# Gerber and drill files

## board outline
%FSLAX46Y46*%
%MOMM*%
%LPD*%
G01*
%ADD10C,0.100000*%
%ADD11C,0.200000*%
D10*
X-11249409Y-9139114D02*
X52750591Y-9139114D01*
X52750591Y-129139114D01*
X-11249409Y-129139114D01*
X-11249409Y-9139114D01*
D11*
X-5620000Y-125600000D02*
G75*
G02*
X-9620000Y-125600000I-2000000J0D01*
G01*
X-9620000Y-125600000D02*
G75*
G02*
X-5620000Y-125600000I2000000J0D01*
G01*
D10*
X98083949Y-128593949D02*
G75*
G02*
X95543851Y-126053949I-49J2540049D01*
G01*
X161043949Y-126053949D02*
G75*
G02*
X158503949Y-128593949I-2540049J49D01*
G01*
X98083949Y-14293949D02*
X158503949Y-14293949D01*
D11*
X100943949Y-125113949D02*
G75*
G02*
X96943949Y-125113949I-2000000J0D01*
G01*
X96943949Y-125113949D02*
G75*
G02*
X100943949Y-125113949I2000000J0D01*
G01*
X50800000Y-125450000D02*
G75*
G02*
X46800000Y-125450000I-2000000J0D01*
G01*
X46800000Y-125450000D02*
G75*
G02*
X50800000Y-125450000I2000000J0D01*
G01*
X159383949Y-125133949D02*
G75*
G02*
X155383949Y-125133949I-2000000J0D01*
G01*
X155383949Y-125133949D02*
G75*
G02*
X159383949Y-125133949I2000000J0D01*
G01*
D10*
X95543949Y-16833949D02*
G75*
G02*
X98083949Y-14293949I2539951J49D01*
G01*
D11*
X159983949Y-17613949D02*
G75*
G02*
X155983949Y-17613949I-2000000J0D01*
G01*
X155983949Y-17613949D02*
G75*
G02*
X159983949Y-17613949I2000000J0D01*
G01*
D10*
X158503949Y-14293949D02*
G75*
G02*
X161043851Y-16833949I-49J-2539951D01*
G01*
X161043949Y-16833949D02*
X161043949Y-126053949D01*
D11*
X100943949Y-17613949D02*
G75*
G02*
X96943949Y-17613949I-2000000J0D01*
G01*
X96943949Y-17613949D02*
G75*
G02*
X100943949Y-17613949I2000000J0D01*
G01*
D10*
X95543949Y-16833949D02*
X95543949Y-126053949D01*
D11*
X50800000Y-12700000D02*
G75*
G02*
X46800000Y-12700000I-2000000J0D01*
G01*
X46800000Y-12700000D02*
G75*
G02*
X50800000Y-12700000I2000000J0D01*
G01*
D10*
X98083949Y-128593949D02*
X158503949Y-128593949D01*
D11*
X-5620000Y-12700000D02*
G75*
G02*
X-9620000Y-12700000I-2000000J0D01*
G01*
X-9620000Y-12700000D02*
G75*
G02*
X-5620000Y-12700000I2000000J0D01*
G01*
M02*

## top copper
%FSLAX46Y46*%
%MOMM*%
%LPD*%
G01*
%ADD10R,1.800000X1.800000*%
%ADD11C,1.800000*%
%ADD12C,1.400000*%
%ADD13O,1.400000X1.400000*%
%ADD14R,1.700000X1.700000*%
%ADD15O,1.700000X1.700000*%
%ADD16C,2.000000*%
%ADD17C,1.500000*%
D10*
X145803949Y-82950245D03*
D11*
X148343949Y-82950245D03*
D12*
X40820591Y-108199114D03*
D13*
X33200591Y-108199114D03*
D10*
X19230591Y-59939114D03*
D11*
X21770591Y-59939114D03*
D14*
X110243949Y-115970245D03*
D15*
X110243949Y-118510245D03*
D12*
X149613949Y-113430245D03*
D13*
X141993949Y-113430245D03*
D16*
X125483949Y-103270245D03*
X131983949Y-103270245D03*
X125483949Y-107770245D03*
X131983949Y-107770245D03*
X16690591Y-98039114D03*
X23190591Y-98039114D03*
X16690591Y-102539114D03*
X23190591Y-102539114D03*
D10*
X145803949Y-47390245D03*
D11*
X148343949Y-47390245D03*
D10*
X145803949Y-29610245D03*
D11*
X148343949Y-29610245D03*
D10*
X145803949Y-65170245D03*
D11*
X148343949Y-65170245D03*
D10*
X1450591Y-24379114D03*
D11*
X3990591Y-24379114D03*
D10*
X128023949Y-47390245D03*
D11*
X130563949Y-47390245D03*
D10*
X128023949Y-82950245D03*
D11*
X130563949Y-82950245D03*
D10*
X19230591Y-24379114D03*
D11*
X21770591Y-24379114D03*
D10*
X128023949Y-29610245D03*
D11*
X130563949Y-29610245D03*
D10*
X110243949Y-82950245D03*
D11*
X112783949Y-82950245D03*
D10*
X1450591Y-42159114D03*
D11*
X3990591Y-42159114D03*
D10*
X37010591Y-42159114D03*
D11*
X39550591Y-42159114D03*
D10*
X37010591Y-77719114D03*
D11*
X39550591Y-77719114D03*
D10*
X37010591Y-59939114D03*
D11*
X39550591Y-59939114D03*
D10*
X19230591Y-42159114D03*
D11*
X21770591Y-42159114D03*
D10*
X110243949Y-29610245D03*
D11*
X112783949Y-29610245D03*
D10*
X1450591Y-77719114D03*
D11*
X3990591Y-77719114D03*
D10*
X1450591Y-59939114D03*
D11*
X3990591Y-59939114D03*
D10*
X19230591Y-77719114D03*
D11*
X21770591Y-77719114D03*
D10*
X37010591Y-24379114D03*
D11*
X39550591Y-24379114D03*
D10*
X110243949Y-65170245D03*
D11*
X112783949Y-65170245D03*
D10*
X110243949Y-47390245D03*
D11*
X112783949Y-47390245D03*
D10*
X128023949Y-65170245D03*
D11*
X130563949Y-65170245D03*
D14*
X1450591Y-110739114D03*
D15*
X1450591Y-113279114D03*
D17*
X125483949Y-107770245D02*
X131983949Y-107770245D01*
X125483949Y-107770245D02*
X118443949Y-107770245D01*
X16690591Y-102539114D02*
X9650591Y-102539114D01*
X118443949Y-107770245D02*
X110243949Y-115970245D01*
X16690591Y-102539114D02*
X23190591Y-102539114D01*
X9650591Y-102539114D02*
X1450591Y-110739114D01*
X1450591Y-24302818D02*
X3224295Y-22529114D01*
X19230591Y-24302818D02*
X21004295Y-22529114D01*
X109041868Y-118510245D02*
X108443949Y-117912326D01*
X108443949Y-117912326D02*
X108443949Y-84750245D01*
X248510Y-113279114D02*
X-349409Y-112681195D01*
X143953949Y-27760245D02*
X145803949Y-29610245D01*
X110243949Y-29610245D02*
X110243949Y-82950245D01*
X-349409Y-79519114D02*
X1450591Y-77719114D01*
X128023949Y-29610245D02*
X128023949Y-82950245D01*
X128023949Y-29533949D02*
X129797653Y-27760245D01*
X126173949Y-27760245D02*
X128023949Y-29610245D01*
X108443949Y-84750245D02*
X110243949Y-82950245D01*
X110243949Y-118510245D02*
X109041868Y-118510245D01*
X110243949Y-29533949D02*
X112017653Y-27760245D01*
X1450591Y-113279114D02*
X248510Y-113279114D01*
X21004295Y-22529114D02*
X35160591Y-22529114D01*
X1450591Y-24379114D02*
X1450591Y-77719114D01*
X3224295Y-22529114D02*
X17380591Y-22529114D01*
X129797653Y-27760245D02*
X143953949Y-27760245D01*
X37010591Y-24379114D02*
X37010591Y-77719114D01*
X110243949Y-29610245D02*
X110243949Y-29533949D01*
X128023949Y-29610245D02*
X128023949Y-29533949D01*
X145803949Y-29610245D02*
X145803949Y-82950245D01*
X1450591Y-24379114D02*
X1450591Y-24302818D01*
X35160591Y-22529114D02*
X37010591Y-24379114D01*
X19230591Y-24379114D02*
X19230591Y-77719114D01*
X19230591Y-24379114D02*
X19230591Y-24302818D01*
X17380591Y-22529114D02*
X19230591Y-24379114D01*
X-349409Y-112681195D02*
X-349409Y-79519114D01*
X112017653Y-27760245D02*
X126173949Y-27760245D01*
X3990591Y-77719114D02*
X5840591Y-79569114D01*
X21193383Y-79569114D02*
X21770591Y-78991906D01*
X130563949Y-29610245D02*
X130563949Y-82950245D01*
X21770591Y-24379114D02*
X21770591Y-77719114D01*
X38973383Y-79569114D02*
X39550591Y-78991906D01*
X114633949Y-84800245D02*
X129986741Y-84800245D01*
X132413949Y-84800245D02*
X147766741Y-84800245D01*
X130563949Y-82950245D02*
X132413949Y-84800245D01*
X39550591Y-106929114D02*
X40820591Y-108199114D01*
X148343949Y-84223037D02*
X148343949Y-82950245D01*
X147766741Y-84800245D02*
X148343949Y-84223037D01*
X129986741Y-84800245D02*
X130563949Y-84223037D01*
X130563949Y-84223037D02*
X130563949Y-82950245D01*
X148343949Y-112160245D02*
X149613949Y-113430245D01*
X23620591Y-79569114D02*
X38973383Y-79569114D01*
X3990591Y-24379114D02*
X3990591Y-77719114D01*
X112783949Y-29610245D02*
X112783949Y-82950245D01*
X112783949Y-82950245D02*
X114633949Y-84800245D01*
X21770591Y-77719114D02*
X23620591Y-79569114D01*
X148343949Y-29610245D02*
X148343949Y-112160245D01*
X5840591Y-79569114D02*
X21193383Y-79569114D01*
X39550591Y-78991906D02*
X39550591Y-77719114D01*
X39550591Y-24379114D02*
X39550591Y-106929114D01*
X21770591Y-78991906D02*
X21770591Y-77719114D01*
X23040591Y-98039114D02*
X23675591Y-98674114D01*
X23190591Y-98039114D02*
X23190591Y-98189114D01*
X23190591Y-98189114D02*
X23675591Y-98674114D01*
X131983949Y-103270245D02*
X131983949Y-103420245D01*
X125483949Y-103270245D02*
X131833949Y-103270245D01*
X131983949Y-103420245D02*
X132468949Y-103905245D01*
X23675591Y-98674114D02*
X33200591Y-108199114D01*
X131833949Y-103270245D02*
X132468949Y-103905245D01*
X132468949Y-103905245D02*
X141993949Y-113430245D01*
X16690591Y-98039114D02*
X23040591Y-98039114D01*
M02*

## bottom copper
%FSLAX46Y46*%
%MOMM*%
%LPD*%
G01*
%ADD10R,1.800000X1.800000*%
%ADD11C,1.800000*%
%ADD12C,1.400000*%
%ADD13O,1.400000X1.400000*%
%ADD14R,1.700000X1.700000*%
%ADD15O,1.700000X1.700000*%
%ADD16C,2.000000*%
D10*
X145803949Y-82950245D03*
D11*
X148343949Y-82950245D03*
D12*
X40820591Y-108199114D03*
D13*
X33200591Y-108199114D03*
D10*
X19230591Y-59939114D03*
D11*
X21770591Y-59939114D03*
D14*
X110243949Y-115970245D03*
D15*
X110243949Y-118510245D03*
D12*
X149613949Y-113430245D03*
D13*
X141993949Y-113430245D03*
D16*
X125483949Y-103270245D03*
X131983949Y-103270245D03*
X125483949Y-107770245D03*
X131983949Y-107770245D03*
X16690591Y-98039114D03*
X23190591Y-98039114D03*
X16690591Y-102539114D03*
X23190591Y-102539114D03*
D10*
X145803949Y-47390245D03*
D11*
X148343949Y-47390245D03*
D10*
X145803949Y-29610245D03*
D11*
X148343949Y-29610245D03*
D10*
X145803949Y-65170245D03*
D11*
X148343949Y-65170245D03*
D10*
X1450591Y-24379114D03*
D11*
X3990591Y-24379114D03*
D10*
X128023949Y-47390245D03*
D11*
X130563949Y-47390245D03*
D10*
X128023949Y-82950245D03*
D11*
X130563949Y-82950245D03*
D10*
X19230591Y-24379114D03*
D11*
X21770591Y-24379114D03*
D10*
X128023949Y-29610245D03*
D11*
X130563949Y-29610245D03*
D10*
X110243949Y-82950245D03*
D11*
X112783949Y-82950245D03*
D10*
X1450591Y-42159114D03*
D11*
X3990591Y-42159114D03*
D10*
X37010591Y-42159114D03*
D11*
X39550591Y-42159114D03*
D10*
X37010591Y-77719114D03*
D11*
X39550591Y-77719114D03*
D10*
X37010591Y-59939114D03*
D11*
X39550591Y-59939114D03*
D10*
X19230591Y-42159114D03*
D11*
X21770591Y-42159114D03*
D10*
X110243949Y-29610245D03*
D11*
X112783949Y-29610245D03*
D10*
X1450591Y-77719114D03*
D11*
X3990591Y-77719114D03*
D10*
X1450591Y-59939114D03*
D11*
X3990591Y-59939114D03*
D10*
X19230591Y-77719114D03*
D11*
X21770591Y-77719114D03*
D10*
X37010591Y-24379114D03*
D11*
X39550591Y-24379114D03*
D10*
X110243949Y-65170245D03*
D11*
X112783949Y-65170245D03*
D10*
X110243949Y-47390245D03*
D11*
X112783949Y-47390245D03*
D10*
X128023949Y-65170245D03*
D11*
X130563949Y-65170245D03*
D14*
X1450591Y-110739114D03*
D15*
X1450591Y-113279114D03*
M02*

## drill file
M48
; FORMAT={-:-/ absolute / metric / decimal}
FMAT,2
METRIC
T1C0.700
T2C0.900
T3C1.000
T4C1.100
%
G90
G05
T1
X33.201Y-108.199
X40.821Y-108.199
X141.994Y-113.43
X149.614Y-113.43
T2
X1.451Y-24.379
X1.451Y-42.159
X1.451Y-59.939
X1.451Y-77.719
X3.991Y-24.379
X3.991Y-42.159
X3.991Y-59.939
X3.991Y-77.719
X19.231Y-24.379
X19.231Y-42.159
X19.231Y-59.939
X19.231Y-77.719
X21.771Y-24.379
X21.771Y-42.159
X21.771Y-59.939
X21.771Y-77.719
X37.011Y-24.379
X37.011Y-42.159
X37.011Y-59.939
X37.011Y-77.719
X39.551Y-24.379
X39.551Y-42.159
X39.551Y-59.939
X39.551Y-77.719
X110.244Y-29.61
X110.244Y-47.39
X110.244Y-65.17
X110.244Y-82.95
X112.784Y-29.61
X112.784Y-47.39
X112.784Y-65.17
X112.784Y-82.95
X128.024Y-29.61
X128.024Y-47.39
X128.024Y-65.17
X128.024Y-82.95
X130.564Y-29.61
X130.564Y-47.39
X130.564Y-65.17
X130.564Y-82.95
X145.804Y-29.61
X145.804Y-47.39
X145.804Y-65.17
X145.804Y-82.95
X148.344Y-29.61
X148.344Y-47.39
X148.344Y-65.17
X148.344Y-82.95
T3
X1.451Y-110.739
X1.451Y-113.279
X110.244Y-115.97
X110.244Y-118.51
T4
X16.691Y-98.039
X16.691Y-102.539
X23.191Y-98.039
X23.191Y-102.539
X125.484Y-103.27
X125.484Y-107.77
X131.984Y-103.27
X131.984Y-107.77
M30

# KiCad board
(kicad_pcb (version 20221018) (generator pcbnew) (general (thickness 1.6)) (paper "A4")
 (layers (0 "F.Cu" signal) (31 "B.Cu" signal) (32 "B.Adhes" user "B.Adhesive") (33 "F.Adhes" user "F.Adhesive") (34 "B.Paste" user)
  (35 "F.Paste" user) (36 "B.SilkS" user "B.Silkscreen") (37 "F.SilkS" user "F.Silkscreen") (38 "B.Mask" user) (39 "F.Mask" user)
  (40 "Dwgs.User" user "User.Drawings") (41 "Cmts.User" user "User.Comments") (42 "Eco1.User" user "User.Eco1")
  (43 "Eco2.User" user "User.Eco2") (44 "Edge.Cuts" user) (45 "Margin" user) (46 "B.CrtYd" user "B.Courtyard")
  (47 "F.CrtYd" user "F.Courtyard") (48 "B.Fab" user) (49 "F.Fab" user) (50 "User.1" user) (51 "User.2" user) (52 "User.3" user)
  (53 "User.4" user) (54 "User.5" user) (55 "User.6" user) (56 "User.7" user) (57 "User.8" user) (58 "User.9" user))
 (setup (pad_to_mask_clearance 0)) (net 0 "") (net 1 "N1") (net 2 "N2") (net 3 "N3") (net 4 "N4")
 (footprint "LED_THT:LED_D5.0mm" (layer "F.Cu") (at 145.803949 82.950245)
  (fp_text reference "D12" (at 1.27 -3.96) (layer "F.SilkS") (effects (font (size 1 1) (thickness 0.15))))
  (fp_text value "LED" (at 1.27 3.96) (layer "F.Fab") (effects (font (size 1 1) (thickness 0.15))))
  (pad "1" thru_hole rect (at 0 0) (size 1.8 1.8) (drill 0.9) (layers "*.Cu" "*.Mask") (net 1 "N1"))
  (pad "2" thru_hole circle (at 2.54 0) (size 1.8 1.8) (drill 0.9) (layers "*.Cu" "*.Mask") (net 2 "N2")))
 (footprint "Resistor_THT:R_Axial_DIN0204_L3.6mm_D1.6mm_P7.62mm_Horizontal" (layer "F.Cu") (at 40.820591 108.199114 180)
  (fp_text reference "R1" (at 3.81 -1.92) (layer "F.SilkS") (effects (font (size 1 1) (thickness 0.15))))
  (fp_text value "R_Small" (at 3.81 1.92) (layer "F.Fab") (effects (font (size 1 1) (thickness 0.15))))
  (pad "1" thru_hole circle (at 0 0 180) (size 1.4 1.4) (drill 0.7) (layers "*.Cu" "*.Mask") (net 2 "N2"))
  (pad "2" thru_hole oval (at 7.62 0 180) (size 1.4 1.4) (drill 0.7) (layers "*.Cu" "*.Mask") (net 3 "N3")))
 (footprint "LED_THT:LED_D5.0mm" (layer "F.Cu") (at 19.230591 59.939114)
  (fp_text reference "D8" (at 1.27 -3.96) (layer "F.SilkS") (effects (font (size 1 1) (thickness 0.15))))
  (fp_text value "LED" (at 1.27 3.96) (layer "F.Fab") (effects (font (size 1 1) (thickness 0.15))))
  (pad "1" thru_hole rect (at 0 0) (size 1.8 1.8) (drill 0.9) (layers "*.Cu" "*.Mask") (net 1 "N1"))
  (pad "2" thru_hole circle (at 2.54 0) (size 1.8 1.8) (drill 0.9) (layers "*.Cu" "*.Mask") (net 2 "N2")))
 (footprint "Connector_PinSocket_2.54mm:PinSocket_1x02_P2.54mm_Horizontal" (layer "F.Cu") (at 110.243949 115.970245)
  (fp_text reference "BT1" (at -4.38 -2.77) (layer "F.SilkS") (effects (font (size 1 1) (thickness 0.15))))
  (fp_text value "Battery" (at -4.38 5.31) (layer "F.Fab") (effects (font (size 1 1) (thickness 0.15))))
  (pad "1" thru_hole rect (at 0 0) (size 1.7 1.7) (drill 1) (layers "*.Cu" "*.Mask") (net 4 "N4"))
  (pad "2" thru_hole oval (at 0 2.54) (size 1.7 1.7) (drill 1) (layers "*.Cu" "*.Mask") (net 1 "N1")))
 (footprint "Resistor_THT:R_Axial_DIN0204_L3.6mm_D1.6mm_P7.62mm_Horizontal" (layer "F.Cu") (at 149.613949 113.430245 180)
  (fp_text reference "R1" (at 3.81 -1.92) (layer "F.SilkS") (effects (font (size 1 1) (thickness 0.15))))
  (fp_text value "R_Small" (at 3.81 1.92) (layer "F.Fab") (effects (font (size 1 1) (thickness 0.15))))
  (pad "1" thru_hole circle (at 0 0 180) (size 1.4 1.4) (drill 0.7) (layers "*.Cu" "*.Mask") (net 2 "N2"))
  (pad "2" thru_hole oval (at 7.62 0 180) (size 1.4 1.4) (drill 0.7) (layers "*.Cu" "*.Mask") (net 3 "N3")))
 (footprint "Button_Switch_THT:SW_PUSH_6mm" (layer "F.Cu") (at 125.483949 103.270245)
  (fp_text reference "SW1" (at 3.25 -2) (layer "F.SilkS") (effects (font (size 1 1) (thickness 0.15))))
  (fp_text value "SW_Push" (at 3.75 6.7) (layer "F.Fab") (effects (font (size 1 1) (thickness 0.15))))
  (pad "1" thru_hole circle (at 0 0 90) (size 2 2) (drill 1.1) (layers "*.Cu" "*.Mask") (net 3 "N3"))
  (pad "1" thru_hole circle (at 6.5 0 90) (size 2 2) (drill 1.1) (layers "*.Cu" "*.Mask") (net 3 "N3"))
  (pad "2" thru_hole circle (at 0 4.5 90) (size 2 2) (drill 1.1) (layers "*.Cu" "*.Mask") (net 4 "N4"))
  (pad "2" thru_hole circle (at 6.5 4.5 90) (size 2 2) (drill 1.1) (layers "*.Cu" "*.Mask") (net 4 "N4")))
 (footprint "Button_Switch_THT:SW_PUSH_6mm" (layer "F.Cu") (at 16.690591 98.039114)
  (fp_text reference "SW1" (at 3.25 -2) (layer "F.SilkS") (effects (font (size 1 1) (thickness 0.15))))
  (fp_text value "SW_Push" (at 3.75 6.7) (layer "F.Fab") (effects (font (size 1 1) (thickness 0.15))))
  (pad "1" thru_hole circle (at 0 0 90) (size 2 2) (drill 1.1) (layers "*.Cu" "*.Mask") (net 3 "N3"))
  (pad "1" thru_hole circle (at 6.5 0 90) (size 2 2) (drill 1.1) (layers "*.Cu" "*.Mask") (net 3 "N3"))
  (pad "2" thru_hole circle (at 0 4.5 90) (size 2 2) (drill 1.1) (layers "*.Cu" "*.Mask") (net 4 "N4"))
  (pad "2" thru_hole circle (at 6.5 4.5 90) (size 2 2) (drill 1.1) (layers "*.Cu" "*.Mask") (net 4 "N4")))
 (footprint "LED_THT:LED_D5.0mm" (layer "F.Cu") (at 145.803949 47.390245)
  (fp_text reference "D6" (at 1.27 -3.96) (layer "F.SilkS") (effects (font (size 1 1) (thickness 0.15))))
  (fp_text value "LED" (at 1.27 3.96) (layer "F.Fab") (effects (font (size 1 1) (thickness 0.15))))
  (pad "1" thru_hole rect (at 0 0) (size 1.8 1.8) (drill 0.9) (layers "*.Cu" "*.Mask") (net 1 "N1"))
  (pad "2" thru_hole circle (at 2.54 0) (size 1.8 1.8) (drill 0.9) (layers "*.Cu" "*.Mask") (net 2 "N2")))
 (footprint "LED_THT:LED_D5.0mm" (layer "F.Cu") (at 145.803949 29.610245)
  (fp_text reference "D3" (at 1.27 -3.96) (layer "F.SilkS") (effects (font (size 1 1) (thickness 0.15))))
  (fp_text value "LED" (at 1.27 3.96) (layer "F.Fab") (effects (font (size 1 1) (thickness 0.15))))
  (pad "1" thru_hole rect (at 0 0) (size 1.8 1.8) (drill 0.9) (layers "*.Cu" "*.Mask") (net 1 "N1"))
  (pad "2" thru_hole circle (at 2.54 0) (size 1.8 1.8) (drill 0.9) (layers "*.Cu" "*.Mask") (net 2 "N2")))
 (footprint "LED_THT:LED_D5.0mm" (layer "F.Cu") (at 145.803949 65.170245)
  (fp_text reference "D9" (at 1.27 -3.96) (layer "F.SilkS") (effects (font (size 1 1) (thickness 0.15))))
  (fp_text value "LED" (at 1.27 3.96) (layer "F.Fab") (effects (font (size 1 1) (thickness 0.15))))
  (pad "1" thru_hole rect (at 0 0) (size 1.8 1.8) (drill 0.9) (layers "*.Cu" "*.Mask") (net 1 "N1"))
  (pad "2" thru_hole circle (at 2.54 0) (size 1.8 1.8) (drill 0.9) (layers "*.Cu" "*.Mask") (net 2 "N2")))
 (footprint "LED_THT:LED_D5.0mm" (layer "F.Cu") (at 1.450591 24.379114)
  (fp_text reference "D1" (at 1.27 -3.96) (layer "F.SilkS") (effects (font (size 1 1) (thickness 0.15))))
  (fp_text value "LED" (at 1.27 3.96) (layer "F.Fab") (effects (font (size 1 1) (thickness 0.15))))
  (pad "1" thru_hole rect (at 0 0) (size 1.8 1.8) (drill 0.9) (layers "*.Cu" "*.Mask") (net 1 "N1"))
  (pad "2" thru_hole circle (at 2.54 0) (size 1.8 1.8) (drill 0.9) (layers "*.Cu" "*.Mask") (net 2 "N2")))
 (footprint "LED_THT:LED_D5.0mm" (layer "F.Cu") (at 128.023949 47.390245)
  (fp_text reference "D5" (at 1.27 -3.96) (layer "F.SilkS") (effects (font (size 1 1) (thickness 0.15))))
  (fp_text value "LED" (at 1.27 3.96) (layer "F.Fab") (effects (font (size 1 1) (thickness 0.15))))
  (pad "1" thru_hole rect (at 0 0) (size 1.8 1.8) (drill 0.9) (layers "*.Cu" "*.Mask") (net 1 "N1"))
  (pad "2" thru_hole circle (at 2.54 0) (size 1.8 1.8) (drill 0.9) (layers "*.Cu" "*.Mask") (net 2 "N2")))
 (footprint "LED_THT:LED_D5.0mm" (layer "F.Cu") (at 128.023949 82.950245)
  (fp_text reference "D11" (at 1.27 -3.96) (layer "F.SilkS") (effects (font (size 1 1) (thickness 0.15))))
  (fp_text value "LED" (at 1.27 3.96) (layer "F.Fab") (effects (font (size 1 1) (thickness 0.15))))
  (pad "1" thru_hole rect (at 0 0) (size 1.8 1.8) (drill 0.9) (layers "*.Cu" "*.Mask") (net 1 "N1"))
  (pad "2" thru_hole circle (at 2.54 0) (size 1.8 1.8) (drill 0.9) (layers "*.Cu" "*.Mask") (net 2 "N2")))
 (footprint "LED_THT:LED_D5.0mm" (layer "F.Cu") (at 19.230591 24.379114)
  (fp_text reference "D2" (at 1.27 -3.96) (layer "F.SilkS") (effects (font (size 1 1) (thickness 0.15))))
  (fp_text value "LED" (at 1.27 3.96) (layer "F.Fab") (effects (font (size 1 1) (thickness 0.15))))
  (pad "1" thru_hole rect (at 0 0) (size 1.8 1.8) (drill 0.9) (layers "*.Cu" "*.Mask") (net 1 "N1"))
  (pad "2" thru_hole circle (at 2.54 0) (size 1.8 1.8) (drill 0.9) (layers "*.Cu" "*.Mask") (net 2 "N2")))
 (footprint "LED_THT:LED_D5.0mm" (layer "F.Cu") (at 128.023949 29.610245)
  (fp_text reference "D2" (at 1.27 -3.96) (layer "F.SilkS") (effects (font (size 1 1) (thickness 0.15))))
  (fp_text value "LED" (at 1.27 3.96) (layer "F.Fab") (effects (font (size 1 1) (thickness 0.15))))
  (pad "1" thru_hole rect (at 0 0) (size 1.8 1.8) (drill 0.9) (layers "*.Cu" "*.Mask") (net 1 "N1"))
  (pad "2" thru_hole circle (at 2.54 0) (size 1.8 1.8) (drill 0.9) (layers "*.Cu" "*.Mask") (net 2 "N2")))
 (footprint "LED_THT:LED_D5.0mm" (layer "F.Cu") (at 110.243949 82.950245)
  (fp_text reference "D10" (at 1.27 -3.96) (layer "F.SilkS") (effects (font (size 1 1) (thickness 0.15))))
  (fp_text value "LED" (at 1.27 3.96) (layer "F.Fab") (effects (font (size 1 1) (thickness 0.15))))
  (pad "1" thru_hole rect (at 0 0) (size 1.8 1.8) (drill 0.9) (layers "*.Cu" "*.Mask") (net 1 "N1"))
  (pad "2" thru_hole circle (at 2.54 0) (size 1.8 1.8) (drill 0.9) (layers "*.Cu" "*.Mask") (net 2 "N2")))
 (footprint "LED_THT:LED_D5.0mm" (layer "F.Cu") (at 1.450591 42.159114)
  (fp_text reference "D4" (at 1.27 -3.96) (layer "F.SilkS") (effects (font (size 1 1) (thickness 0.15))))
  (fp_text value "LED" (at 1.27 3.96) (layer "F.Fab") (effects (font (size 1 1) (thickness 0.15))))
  (pad "1" thru_hole rect (at 0 0) (size 1.8 1.8) (drill 0.9) (layers "*.Cu" "*.Mask") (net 1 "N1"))
  (pad "2" thru_hole circle (at 2.54 0) (size 1.8 1.8) (drill 0.9) (layers "*.Cu" "*.Mask") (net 2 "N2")))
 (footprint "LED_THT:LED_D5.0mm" (layer "F.Cu") (at 37.010591 42.159114)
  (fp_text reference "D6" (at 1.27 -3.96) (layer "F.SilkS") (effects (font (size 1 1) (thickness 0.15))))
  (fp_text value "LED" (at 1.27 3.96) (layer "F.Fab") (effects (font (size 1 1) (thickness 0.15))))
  (pad "1" thru_hole rect (at 0 0) (size 1.8 1.8) (drill 0.9) (layers "*.Cu" "*.Mask") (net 1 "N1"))
  (pad "2" thru_hole circle (at 2.54 0) (size 1.8 1.8) (drill 0.9) (layers "*.Cu" "*.Mask") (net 2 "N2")))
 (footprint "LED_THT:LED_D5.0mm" (layer "F.Cu") (at 37.010591 77.719114)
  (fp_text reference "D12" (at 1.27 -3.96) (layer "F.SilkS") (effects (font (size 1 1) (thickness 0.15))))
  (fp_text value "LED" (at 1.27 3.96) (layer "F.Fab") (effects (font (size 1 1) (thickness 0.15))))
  (pad "1" thru_hole rect (at 0 0) (size 1.8 1.8) (drill 0.9) (layers "*.Cu" "*.Mask") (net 1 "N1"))
  (pad "2" thru_hole circle (at 2.54 0) (size 1.8 1.8) (drill 0.9) (layers "*.Cu" "*.Mask") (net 2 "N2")))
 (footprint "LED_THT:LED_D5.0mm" (layer "F.Cu") (at 37.010591 59.939114)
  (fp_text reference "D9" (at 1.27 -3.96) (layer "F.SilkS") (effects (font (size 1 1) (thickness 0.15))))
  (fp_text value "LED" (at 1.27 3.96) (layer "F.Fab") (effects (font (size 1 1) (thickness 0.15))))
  (pad "1" thru_hole rect (at 0 0) (size 1.8 1.8) (drill 0.9) (layers "*.Cu" "*.Mask") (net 1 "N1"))
  (pad "2" thru_hole circle (at 2.54 0) (size 1.8 1.8) (drill 0.9) (layers "*.Cu" "*.Mask") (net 2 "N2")))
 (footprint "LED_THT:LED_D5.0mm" (layer "F.Cu") (at 19.230591 42.159114)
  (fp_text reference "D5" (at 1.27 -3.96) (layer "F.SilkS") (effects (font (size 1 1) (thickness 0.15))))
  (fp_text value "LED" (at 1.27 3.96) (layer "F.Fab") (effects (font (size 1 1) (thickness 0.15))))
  (pad "1" thru_hole rect (at 0 0) (size 1.8 1.8) (drill 0.9) (layers "*.Cu" "*.Mask") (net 1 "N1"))
  (pad "2" thru_hole circle (at 2.54 0) (size 1.8 1.8) (drill 0.9) (layers "*.Cu" "*.Mask") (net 2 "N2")))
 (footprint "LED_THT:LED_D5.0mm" (layer "F.Cu") (at 110.243949 29.610245)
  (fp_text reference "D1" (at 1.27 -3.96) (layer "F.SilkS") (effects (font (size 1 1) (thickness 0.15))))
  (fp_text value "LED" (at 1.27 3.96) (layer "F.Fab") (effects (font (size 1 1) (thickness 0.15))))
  (pad "1" thru_hole rect (at 0 0) (size 1.8 1.8) (drill 0.9) (layers "*.Cu" "*.Mask") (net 1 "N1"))
  (pad "2" thru_hole circle (at 2.54 0) (size 1.8 1.8) (drill 0.9) (layers "*.Cu" "*.Mask") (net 2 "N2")))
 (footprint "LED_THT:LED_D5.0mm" (layer "F.Cu") (at 1.450591 77.719114)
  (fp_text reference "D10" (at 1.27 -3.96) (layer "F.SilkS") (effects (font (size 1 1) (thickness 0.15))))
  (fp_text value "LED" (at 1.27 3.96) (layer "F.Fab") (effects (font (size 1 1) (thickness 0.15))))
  (pad "1" thru_hole rect (at 0 0) (size 1.8 1.8) (drill 0.9) (layers "*.Cu" "*.Mask") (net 1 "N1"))
  (pad "2" thru_hole circle (at 2.54 0) (size 1.8 1.8) (drill 0.9) (layers "*.Cu" "*.Mask") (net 2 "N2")))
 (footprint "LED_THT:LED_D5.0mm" (layer "F.Cu") (at 1.450591 59.939114)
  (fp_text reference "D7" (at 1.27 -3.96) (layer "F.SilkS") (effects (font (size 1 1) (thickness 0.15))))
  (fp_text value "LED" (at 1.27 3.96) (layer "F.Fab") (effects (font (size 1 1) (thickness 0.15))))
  (pad "1" thru_hole rect (at 0 0) (size 1.8 1.8) (drill 0.9) (layers "*.Cu" "*.Mask") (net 1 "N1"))
  (pad "2" thru_hole circle (at 2.54 0) (size 1.8 1.8) (drill 0.9) (layers "*.Cu" "*.Mask") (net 2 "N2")))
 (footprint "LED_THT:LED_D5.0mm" (layer "F.Cu") (at 19.230591 77.719114)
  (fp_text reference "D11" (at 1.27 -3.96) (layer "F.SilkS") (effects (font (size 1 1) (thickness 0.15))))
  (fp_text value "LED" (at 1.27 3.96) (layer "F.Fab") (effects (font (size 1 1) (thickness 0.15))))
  (pad "1" thru_hole rect (at 0 0) (size 1.8 1.8) (drill 0.9) (layers "*.Cu" "*.Mask") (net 1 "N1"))
  (pad "2" thru_hole circle (at 2.54 0) (size 1.8 1.8) (drill 0.9) (layers "*.Cu" "*.Mask") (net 2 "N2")))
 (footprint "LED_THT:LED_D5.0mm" (layer "F.Cu") (at 37.010591 24.379114)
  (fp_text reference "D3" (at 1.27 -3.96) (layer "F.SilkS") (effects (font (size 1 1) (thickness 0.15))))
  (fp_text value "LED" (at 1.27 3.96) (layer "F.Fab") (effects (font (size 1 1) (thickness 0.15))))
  (pad "1" thru_hole rect (at 0 0) (size 1.8 1.8) (drill 0.9) (layers "*.Cu" "*.Mask") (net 1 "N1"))
  (pad "2" thru_hole circle (at 2.54 0) (size 1.8 1.8) (drill 0.9) (layers "*.Cu" "*.Mask") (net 2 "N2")))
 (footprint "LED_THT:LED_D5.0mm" (layer "F.Cu") (at 110.243949 65.170245)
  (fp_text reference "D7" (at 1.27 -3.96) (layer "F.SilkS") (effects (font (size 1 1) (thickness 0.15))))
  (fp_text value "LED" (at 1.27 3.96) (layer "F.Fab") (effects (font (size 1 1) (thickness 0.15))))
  (pad "1" thru_hole rect (at 0 0) (size 1.8 1.8) (drill 0.9) (layers "*.Cu" "*.Mask") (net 1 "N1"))
  (pad "2" thru_hole circle (at 2.54 0) (size 1.8 1.8) (drill 0.9) (layers "*.Cu" "*.Mask") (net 2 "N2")))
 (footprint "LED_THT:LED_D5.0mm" (layer "F.Cu") (at 110.243949 47.390245)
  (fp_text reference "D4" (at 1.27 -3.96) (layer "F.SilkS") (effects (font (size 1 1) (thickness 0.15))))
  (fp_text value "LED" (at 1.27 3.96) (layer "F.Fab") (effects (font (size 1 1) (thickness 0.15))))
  (pad "1" thru_hole rect (at 0 0) (size 1.8 1.8) (drill 0.9) (layers "*.Cu" "*.Mask") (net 1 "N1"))
  (pad "2" thru_hole circle (at 2.54 0) (size 1.8 1.8) (drill 0.9) (layers "*.Cu" "*.Mask") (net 2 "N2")))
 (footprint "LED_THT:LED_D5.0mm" (layer "F.Cu") (at 128.023949 65.170245)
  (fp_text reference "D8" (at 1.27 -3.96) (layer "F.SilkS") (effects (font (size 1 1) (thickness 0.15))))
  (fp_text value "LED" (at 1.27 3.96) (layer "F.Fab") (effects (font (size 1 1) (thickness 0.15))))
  (pad "1" thru_hole rect (at 0 0) (size 1.8 1.8) (drill 0.9) (layers "*.Cu" "*.Mask") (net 1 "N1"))
  (pad "2" thru_hole circle (at 2.54 0) (size 1.8 1.8) (drill 0.9) (layers "*.Cu" "*.Mask") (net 2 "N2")))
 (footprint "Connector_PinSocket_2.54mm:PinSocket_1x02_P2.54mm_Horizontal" (layer "F.Cu") (at 1.450591 110.739114)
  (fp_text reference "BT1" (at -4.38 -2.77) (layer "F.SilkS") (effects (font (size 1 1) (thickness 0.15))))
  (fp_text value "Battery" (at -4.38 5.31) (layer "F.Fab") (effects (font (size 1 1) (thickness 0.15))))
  (pad "1" thru_hole rect (at 0 0) (size 1.7 1.7) (drill 1) (layers "*.Cu" "*.Mask") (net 4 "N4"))
  (pad "2" thru_hole oval (at 0 2.54) (size 1.7 1.7) (drill 1) (layers "*.Cu" "*.Mask") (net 1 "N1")))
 (gr_rect (start -11.249409 9.139114) (end 52.750591 129.139114) (stroke (width 0.1) (type default)) (fill none) (layer "Edge.Cuts"))
 (gr_circle (center -7.62 125.6) (end -5.62 125.6) (stroke (width 0.2) (type default)) (fill none) (layer "Edge.Cuts"))
 (gr_arc (start 98.083949 128.593949) (mid 96.287898 127.85) (end 95.543949 126.053949) (stroke (width 0.1) (type default))
  (layer "Edge.Cuts"))
 (gr_arc (start 161.043949 126.053949) (mid 160.3 127.85) (end 158.503949 128.593949) (stroke (width 0.1) (type default))
  (layer "Edge.Cuts"))
 (gr_line (start 98.083949 14.293949) (end 158.503949 14.293949) (stroke (width 0.1) (type default)) (layer "Edge.Cuts"))
 (gr_circle (center 98.943949 125.113949) (end 96.943949 125.113949) (stroke (width 0.2) (type default)) (fill none) (layer "Edge.Cuts"))
 (gr_circle (center 48.8 125.45) (end 50.8 125.45) (stroke (width 0.2) (type default)) (fill none) (layer "Edge.Cuts"))
 (gr_circle (center 157.383949 125.133949) (end 155.383949 125.133949) (stroke (width 0.2) (type default)) (fill none) (layer "Edge.Cuts"))
 (gr_arc (start 95.543949 16.833949) (mid 96.287898 15.037898) (end 98.083949 14.293949) (stroke (width 0.1) (type default))
  (layer "Edge.Cuts"))
 (gr_circle (center 157.983949 17.613949) (end 155.983949 17.613949) (stroke (width 0.2) (type default)) (fill none) (layer "Edge.Cuts"))
 (gr_arc (start 158.503949 14.293949) (mid 160.3 15.037898) (end 161.043949 16.833949) (stroke (width 0.1) (type default))
  (layer "Edge.Cuts"))
 (gr_line (start 161.043949 16.833949) (end 161.043949 126.053949) (stroke (width 0.1) (type default)) (layer "Edge.Cuts"))
 (gr_circle (center 98.943949 17.613949) (end 96.943949 17.613949) (stroke (width 0.2) (type default)) (fill none) (layer "Edge.Cuts"))
 (gr_line (start 95.543949 16.833949) (end 95.543949 126.053949) (stroke (width 0.1) (type default)) (layer "Edge.Cuts"))
 (gr_circle (center 48.8 12.7) (end 50.8 12.7) (stroke (width 0.2) (type default)) (fill none) (layer "Edge.Cuts"))
 (gr_line (start 98.083949 128.593949) (end 158.503949 128.593949) (stroke (width 0.1) (type default)) (layer "Edge.Cuts"))
 (gr_circle (center -7.62 12.7) (end -5.62 12.7) (stroke (width 0.2) (type default)) (fill none) (layer "Edge.Cuts"))
 (segment (start 125.483949 107.770245) (end 131.983949 107.770245) (width 1.5) (layer "F.Cu") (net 4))
 (segment (start 125.483949 107.770245) (end 118.443949 107.770245) (width 1.5) (layer "F.Cu") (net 4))
 (segment (start 16.690591 102.539114) (end 9.650591 102.539114) (width 1.5) (layer "F.Cu") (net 4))
 (segment (start 118.443949 107.770245) (end 110.243949 115.970245) (width 1.5) (layer "F.Cu") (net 4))
 (segment (start 16.690591 102.539114) (end 23.190591 102.539114) (width 1.5) (layer "F.Cu") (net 4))
 (segment (start 9.650591 102.539114) (end 1.450591 110.739114) (width 1.5) (layer "F.Cu") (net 4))
 (segment (start 1.450591 24.302818) (end 3.224295 22.529114) (width 1.5) (layer "F.Cu") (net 1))
 (segment (start 19.230591 24.302818) (end 21.004295 22.529114) (width 1.5) (layer "F.Cu") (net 1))
 (segment (start 109.041868 118.510245) (end 108.443949 117.912326) (width 1.5) (layer "F.Cu") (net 1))
 (segment (start 108.443949 117.912326) (end 108.443949 84.750245) (width 1.5) (layer "F.Cu") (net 1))
 (segment (start 0.24851 113.279114) (end -0.349409 112.681195) (width 1.5) (layer "F.Cu") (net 1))
 (segment (start 143.953949 27.760245) (end 145.803949 29.610245) (width 1.5) (layer "F.Cu") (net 1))
 (segment (start 110.243949 29.610245) (end 110.243949 82.950245) (width 1.5) (layer "F.Cu") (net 1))
 (segment (start -0.349409 79.519114) (end 1.450591 77.719114) (width 1.5) (layer "F.Cu") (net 1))
 (segment (start 128.023949 29.610245) (end 128.023949 82.950245) (width 1.5) (layer "F.Cu") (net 1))
 (segment (start 128.023949 29.533949) (end 129.797653 27.760245) (width 1.5) (layer "F.Cu") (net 1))
 (segment (start 126.173949 27.760245) (end 128.023949 29.610245) (width 1.5) (layer "F.Cu") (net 1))
 (segment (start 108.443949 84.750245) (end 110.243949 82.950245) (width 1.5) (layer "F.Cu") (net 1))
 (segment (start 110.243949 118.510245) (end 109.041868 118.510245) (width 1.5) (layer "F.Cu") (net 1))
 (segment (start 110.243949 29.533949) (end 112.017653 27.760245) (width 1.5) (layer "F.Cu") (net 1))
 (segment (start 1.450591 113.279114) (end 0.24851 113.279114) (width 1.5) (layer "F.Cu") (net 1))
 (segment (start 21.004295 22.529114) (end 35.160591 22.529114) (width 1.5) (layer "F.Cu") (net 1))
 (segment (start 1.450591 24.379114) (end 1.450591 77.719114) (width 1.5) (layer "F.Cu") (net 1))
 (segment (start 3.224295 22.529114) (end 17.380591 22.529114) (width 1.5) (layer "F.Cu") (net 1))
 (segment (start 129.797653 27.760245) (end 143.953949 27.760245) (width 1.5) (layer "F.Cu") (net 1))
 (segment (start 37.010591 24.379114) (end 37.010591 77.719114) (width 1.5) (layer "F.Cu") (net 1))
 (segment (start 110.243949 29.610245) (end 110.243949 29.533949) (width 1.5) (layer "F.Cu") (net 1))
 (segment (start 128.023949 29.610245) (end 128.023949 29.533949) (width 1.5) (layer "F.Cu") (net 1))
 (segment (start 145.803949 29.610245) (end 145.803949 82.950245) (width 1.5) (layer "F.Cu") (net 1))
 (segment (start 1.450591 24.379114) (end 1.450591 24.302818) (width 1.5) (layer "F.Cu") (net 1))
 (segment (start 35.160591 22.529114) (end 37.010591 24.379114) (width 1.5) (layer "F.Cu") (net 1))
 (segment (start 19.230591 24.379114) (end 19.230591 77.719114) (width 1.5) (layer "F.Cu") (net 1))
 (segment (start 19.230591 24.379114) (end 19.230591 24.302818) (width 1.5) (layer "F.Cu") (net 1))
 (segment (start 17.380591 22.529114) (end 19.230591 24.379114) (width 1.5) (layer "F.Cu") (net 1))
 (segment (start -0.349409 112.681195) (end -0.349409 79.519114) (width 1.5) (layer "F.Cu") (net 1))
 (segment (start 112.017653 27.760245) (end 126.173949 27.760245) (width 1.5) (layer "F.Cu") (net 1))
 (segment (start 3.990591 77.719114) (end 5.840591 79.569114) (width 1.5) (layer "F.Cu") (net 2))
 (segment (start 21.193383 79.569114) (end 21.770591 78.991906) (width 1.5) (layer "F.Cu") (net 2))
 (segment (start 130.563949 29.610245) (end 130.563949 82.950245) (width 1.5) (layer "F.Cu") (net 2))
 (segment (start 21.770591 24.379114) (end 21.770591 77.719114) (width 1.5) (layer "F.Cu") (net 2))
 (segment (start 38.973383 79.569114) (end 39.550591 78.991906) (width 1.5) (layer "F.Cu") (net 2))
 (segment (start 114.633949 84.800245) (end 129.986741 84.800245) (width 1.5) (layer "F.Cu") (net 2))
 (segment (start 132.413949 84.800245) (end 147.766741 84.800245) (width 1.5) (layer "F.Cu") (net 2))
 (segment (start 130.563949 82.950245) (end 132.413949 84.800245) (width 1.5) (layer "F.Cu") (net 2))
 (segment (start 39.550591 106.929114) (end 40.820591 108.199114) (width 1.5) (layer "F.Cu") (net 2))
 (segment (start 148.343949 84.223037) (end 148.343949 82.950245) (width 1.5) (layer "F.Cu") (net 2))
 (segment (start 147.766741 84.800245) (end 148.343949 84.223037) (width 1.5) (layer "F.Cu") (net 2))
 (segment (start 129.986741 84.800245) (end 130.563949 84.223037) (width 1.5) (layer "F.Cu") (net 2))
 (segment (start 130.563949 84.223037) (end 130.563949 82.950245) (width 1.5) (layer "F.Cu") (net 2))
 (segment (start 148.343949 112.160245) (end 149.613949 113.430245) (width 1.5) (layer "F.Cu") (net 2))
 (segment (start 23.620591 79.569114) (end 38.973383 79.569114) (width 1.5) (layer "F.Cu") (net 2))
 (segment (start 3.990591 24.379114) (end 3.990591 77.719114) (width 1.5) (layer "F.Cu") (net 2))
 (segment (start 112.783949 29.610245) (end 112.783949 82.950245) (width 1.5) (layer "F.Cu") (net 2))
 (segment (start 112.783949 82.950245) (end 114.633949 84.800245) (width 1.5) (layer "F.Cu") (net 2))
 (segment (start 21.770591 77.719114) (end 23.620591 79.569114) (width 1.5) (layer "F.Cu") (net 2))
 (segment (start 148.343949 29.610245) (end 148.343949 112.160245) (width 1.5) (layer "F.Cu") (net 2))
 (segment (start 5.840591 79.569114) (end 21.193383 79.569114) (width 1.5) (layer "F.Cu") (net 2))
 (segment (start 39.550591 78.991906) (end 39.550591 77.719114) (width 1.5) (layer "F.Cu") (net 2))
 (segment (start 39.550591 24.379114) (end 39.550591 106.929114) (width 1.5) (layer "F.Cu") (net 2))
 (segment (start 21.770591 78.991906) (end 21.770591 77.719114) (width 1.5) (layer "F.Cu") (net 2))
 (segment (start 23.040591 98.039114) (end 23.675591 98.674114) (width 1.5) (layer "F.Cu") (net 3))
 (segment (start 23.190591 98.039114) (end 23.190591 98.189114) (width 1.5) (layer "F.Cu") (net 3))
 (segment (start 23.190591 98.189114) (end 23.675591 98.674114) (width 1.5) (layer "F.Cu") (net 3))
 (segment (start 131.983949 103.270245) (end 131.983949 103.420245) (width 1.5) (layer "F.Cu") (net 3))
 (segment (start 125.483949 103.270245) (end 131.833949 103.270245) (width 1.5) (layer "F.Cu") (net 3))
 (segment (start 131.983949 103.420245) (end 132.468949 103.905245) (width 1.5) (layer "F.Cu") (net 3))
 (segment (start 23.675591 98.674114) (end 33.200591 108.199114) (width 1.5) (layer "F.Cu") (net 3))
 (segment (start 131.833949 103.270245) (end 132.468949 103.905245) (width 1.5) (layer "F.Cu") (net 3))
 (segment (start 132.468949 103.905245) (end 141.993949 113.430245) (width 1.5) (layer "F.Cu") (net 3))
 (segment (start 16.690591 98.039114) (end 23.040591 98.039114) (width 1.5) (layer "F.Cu") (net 3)))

